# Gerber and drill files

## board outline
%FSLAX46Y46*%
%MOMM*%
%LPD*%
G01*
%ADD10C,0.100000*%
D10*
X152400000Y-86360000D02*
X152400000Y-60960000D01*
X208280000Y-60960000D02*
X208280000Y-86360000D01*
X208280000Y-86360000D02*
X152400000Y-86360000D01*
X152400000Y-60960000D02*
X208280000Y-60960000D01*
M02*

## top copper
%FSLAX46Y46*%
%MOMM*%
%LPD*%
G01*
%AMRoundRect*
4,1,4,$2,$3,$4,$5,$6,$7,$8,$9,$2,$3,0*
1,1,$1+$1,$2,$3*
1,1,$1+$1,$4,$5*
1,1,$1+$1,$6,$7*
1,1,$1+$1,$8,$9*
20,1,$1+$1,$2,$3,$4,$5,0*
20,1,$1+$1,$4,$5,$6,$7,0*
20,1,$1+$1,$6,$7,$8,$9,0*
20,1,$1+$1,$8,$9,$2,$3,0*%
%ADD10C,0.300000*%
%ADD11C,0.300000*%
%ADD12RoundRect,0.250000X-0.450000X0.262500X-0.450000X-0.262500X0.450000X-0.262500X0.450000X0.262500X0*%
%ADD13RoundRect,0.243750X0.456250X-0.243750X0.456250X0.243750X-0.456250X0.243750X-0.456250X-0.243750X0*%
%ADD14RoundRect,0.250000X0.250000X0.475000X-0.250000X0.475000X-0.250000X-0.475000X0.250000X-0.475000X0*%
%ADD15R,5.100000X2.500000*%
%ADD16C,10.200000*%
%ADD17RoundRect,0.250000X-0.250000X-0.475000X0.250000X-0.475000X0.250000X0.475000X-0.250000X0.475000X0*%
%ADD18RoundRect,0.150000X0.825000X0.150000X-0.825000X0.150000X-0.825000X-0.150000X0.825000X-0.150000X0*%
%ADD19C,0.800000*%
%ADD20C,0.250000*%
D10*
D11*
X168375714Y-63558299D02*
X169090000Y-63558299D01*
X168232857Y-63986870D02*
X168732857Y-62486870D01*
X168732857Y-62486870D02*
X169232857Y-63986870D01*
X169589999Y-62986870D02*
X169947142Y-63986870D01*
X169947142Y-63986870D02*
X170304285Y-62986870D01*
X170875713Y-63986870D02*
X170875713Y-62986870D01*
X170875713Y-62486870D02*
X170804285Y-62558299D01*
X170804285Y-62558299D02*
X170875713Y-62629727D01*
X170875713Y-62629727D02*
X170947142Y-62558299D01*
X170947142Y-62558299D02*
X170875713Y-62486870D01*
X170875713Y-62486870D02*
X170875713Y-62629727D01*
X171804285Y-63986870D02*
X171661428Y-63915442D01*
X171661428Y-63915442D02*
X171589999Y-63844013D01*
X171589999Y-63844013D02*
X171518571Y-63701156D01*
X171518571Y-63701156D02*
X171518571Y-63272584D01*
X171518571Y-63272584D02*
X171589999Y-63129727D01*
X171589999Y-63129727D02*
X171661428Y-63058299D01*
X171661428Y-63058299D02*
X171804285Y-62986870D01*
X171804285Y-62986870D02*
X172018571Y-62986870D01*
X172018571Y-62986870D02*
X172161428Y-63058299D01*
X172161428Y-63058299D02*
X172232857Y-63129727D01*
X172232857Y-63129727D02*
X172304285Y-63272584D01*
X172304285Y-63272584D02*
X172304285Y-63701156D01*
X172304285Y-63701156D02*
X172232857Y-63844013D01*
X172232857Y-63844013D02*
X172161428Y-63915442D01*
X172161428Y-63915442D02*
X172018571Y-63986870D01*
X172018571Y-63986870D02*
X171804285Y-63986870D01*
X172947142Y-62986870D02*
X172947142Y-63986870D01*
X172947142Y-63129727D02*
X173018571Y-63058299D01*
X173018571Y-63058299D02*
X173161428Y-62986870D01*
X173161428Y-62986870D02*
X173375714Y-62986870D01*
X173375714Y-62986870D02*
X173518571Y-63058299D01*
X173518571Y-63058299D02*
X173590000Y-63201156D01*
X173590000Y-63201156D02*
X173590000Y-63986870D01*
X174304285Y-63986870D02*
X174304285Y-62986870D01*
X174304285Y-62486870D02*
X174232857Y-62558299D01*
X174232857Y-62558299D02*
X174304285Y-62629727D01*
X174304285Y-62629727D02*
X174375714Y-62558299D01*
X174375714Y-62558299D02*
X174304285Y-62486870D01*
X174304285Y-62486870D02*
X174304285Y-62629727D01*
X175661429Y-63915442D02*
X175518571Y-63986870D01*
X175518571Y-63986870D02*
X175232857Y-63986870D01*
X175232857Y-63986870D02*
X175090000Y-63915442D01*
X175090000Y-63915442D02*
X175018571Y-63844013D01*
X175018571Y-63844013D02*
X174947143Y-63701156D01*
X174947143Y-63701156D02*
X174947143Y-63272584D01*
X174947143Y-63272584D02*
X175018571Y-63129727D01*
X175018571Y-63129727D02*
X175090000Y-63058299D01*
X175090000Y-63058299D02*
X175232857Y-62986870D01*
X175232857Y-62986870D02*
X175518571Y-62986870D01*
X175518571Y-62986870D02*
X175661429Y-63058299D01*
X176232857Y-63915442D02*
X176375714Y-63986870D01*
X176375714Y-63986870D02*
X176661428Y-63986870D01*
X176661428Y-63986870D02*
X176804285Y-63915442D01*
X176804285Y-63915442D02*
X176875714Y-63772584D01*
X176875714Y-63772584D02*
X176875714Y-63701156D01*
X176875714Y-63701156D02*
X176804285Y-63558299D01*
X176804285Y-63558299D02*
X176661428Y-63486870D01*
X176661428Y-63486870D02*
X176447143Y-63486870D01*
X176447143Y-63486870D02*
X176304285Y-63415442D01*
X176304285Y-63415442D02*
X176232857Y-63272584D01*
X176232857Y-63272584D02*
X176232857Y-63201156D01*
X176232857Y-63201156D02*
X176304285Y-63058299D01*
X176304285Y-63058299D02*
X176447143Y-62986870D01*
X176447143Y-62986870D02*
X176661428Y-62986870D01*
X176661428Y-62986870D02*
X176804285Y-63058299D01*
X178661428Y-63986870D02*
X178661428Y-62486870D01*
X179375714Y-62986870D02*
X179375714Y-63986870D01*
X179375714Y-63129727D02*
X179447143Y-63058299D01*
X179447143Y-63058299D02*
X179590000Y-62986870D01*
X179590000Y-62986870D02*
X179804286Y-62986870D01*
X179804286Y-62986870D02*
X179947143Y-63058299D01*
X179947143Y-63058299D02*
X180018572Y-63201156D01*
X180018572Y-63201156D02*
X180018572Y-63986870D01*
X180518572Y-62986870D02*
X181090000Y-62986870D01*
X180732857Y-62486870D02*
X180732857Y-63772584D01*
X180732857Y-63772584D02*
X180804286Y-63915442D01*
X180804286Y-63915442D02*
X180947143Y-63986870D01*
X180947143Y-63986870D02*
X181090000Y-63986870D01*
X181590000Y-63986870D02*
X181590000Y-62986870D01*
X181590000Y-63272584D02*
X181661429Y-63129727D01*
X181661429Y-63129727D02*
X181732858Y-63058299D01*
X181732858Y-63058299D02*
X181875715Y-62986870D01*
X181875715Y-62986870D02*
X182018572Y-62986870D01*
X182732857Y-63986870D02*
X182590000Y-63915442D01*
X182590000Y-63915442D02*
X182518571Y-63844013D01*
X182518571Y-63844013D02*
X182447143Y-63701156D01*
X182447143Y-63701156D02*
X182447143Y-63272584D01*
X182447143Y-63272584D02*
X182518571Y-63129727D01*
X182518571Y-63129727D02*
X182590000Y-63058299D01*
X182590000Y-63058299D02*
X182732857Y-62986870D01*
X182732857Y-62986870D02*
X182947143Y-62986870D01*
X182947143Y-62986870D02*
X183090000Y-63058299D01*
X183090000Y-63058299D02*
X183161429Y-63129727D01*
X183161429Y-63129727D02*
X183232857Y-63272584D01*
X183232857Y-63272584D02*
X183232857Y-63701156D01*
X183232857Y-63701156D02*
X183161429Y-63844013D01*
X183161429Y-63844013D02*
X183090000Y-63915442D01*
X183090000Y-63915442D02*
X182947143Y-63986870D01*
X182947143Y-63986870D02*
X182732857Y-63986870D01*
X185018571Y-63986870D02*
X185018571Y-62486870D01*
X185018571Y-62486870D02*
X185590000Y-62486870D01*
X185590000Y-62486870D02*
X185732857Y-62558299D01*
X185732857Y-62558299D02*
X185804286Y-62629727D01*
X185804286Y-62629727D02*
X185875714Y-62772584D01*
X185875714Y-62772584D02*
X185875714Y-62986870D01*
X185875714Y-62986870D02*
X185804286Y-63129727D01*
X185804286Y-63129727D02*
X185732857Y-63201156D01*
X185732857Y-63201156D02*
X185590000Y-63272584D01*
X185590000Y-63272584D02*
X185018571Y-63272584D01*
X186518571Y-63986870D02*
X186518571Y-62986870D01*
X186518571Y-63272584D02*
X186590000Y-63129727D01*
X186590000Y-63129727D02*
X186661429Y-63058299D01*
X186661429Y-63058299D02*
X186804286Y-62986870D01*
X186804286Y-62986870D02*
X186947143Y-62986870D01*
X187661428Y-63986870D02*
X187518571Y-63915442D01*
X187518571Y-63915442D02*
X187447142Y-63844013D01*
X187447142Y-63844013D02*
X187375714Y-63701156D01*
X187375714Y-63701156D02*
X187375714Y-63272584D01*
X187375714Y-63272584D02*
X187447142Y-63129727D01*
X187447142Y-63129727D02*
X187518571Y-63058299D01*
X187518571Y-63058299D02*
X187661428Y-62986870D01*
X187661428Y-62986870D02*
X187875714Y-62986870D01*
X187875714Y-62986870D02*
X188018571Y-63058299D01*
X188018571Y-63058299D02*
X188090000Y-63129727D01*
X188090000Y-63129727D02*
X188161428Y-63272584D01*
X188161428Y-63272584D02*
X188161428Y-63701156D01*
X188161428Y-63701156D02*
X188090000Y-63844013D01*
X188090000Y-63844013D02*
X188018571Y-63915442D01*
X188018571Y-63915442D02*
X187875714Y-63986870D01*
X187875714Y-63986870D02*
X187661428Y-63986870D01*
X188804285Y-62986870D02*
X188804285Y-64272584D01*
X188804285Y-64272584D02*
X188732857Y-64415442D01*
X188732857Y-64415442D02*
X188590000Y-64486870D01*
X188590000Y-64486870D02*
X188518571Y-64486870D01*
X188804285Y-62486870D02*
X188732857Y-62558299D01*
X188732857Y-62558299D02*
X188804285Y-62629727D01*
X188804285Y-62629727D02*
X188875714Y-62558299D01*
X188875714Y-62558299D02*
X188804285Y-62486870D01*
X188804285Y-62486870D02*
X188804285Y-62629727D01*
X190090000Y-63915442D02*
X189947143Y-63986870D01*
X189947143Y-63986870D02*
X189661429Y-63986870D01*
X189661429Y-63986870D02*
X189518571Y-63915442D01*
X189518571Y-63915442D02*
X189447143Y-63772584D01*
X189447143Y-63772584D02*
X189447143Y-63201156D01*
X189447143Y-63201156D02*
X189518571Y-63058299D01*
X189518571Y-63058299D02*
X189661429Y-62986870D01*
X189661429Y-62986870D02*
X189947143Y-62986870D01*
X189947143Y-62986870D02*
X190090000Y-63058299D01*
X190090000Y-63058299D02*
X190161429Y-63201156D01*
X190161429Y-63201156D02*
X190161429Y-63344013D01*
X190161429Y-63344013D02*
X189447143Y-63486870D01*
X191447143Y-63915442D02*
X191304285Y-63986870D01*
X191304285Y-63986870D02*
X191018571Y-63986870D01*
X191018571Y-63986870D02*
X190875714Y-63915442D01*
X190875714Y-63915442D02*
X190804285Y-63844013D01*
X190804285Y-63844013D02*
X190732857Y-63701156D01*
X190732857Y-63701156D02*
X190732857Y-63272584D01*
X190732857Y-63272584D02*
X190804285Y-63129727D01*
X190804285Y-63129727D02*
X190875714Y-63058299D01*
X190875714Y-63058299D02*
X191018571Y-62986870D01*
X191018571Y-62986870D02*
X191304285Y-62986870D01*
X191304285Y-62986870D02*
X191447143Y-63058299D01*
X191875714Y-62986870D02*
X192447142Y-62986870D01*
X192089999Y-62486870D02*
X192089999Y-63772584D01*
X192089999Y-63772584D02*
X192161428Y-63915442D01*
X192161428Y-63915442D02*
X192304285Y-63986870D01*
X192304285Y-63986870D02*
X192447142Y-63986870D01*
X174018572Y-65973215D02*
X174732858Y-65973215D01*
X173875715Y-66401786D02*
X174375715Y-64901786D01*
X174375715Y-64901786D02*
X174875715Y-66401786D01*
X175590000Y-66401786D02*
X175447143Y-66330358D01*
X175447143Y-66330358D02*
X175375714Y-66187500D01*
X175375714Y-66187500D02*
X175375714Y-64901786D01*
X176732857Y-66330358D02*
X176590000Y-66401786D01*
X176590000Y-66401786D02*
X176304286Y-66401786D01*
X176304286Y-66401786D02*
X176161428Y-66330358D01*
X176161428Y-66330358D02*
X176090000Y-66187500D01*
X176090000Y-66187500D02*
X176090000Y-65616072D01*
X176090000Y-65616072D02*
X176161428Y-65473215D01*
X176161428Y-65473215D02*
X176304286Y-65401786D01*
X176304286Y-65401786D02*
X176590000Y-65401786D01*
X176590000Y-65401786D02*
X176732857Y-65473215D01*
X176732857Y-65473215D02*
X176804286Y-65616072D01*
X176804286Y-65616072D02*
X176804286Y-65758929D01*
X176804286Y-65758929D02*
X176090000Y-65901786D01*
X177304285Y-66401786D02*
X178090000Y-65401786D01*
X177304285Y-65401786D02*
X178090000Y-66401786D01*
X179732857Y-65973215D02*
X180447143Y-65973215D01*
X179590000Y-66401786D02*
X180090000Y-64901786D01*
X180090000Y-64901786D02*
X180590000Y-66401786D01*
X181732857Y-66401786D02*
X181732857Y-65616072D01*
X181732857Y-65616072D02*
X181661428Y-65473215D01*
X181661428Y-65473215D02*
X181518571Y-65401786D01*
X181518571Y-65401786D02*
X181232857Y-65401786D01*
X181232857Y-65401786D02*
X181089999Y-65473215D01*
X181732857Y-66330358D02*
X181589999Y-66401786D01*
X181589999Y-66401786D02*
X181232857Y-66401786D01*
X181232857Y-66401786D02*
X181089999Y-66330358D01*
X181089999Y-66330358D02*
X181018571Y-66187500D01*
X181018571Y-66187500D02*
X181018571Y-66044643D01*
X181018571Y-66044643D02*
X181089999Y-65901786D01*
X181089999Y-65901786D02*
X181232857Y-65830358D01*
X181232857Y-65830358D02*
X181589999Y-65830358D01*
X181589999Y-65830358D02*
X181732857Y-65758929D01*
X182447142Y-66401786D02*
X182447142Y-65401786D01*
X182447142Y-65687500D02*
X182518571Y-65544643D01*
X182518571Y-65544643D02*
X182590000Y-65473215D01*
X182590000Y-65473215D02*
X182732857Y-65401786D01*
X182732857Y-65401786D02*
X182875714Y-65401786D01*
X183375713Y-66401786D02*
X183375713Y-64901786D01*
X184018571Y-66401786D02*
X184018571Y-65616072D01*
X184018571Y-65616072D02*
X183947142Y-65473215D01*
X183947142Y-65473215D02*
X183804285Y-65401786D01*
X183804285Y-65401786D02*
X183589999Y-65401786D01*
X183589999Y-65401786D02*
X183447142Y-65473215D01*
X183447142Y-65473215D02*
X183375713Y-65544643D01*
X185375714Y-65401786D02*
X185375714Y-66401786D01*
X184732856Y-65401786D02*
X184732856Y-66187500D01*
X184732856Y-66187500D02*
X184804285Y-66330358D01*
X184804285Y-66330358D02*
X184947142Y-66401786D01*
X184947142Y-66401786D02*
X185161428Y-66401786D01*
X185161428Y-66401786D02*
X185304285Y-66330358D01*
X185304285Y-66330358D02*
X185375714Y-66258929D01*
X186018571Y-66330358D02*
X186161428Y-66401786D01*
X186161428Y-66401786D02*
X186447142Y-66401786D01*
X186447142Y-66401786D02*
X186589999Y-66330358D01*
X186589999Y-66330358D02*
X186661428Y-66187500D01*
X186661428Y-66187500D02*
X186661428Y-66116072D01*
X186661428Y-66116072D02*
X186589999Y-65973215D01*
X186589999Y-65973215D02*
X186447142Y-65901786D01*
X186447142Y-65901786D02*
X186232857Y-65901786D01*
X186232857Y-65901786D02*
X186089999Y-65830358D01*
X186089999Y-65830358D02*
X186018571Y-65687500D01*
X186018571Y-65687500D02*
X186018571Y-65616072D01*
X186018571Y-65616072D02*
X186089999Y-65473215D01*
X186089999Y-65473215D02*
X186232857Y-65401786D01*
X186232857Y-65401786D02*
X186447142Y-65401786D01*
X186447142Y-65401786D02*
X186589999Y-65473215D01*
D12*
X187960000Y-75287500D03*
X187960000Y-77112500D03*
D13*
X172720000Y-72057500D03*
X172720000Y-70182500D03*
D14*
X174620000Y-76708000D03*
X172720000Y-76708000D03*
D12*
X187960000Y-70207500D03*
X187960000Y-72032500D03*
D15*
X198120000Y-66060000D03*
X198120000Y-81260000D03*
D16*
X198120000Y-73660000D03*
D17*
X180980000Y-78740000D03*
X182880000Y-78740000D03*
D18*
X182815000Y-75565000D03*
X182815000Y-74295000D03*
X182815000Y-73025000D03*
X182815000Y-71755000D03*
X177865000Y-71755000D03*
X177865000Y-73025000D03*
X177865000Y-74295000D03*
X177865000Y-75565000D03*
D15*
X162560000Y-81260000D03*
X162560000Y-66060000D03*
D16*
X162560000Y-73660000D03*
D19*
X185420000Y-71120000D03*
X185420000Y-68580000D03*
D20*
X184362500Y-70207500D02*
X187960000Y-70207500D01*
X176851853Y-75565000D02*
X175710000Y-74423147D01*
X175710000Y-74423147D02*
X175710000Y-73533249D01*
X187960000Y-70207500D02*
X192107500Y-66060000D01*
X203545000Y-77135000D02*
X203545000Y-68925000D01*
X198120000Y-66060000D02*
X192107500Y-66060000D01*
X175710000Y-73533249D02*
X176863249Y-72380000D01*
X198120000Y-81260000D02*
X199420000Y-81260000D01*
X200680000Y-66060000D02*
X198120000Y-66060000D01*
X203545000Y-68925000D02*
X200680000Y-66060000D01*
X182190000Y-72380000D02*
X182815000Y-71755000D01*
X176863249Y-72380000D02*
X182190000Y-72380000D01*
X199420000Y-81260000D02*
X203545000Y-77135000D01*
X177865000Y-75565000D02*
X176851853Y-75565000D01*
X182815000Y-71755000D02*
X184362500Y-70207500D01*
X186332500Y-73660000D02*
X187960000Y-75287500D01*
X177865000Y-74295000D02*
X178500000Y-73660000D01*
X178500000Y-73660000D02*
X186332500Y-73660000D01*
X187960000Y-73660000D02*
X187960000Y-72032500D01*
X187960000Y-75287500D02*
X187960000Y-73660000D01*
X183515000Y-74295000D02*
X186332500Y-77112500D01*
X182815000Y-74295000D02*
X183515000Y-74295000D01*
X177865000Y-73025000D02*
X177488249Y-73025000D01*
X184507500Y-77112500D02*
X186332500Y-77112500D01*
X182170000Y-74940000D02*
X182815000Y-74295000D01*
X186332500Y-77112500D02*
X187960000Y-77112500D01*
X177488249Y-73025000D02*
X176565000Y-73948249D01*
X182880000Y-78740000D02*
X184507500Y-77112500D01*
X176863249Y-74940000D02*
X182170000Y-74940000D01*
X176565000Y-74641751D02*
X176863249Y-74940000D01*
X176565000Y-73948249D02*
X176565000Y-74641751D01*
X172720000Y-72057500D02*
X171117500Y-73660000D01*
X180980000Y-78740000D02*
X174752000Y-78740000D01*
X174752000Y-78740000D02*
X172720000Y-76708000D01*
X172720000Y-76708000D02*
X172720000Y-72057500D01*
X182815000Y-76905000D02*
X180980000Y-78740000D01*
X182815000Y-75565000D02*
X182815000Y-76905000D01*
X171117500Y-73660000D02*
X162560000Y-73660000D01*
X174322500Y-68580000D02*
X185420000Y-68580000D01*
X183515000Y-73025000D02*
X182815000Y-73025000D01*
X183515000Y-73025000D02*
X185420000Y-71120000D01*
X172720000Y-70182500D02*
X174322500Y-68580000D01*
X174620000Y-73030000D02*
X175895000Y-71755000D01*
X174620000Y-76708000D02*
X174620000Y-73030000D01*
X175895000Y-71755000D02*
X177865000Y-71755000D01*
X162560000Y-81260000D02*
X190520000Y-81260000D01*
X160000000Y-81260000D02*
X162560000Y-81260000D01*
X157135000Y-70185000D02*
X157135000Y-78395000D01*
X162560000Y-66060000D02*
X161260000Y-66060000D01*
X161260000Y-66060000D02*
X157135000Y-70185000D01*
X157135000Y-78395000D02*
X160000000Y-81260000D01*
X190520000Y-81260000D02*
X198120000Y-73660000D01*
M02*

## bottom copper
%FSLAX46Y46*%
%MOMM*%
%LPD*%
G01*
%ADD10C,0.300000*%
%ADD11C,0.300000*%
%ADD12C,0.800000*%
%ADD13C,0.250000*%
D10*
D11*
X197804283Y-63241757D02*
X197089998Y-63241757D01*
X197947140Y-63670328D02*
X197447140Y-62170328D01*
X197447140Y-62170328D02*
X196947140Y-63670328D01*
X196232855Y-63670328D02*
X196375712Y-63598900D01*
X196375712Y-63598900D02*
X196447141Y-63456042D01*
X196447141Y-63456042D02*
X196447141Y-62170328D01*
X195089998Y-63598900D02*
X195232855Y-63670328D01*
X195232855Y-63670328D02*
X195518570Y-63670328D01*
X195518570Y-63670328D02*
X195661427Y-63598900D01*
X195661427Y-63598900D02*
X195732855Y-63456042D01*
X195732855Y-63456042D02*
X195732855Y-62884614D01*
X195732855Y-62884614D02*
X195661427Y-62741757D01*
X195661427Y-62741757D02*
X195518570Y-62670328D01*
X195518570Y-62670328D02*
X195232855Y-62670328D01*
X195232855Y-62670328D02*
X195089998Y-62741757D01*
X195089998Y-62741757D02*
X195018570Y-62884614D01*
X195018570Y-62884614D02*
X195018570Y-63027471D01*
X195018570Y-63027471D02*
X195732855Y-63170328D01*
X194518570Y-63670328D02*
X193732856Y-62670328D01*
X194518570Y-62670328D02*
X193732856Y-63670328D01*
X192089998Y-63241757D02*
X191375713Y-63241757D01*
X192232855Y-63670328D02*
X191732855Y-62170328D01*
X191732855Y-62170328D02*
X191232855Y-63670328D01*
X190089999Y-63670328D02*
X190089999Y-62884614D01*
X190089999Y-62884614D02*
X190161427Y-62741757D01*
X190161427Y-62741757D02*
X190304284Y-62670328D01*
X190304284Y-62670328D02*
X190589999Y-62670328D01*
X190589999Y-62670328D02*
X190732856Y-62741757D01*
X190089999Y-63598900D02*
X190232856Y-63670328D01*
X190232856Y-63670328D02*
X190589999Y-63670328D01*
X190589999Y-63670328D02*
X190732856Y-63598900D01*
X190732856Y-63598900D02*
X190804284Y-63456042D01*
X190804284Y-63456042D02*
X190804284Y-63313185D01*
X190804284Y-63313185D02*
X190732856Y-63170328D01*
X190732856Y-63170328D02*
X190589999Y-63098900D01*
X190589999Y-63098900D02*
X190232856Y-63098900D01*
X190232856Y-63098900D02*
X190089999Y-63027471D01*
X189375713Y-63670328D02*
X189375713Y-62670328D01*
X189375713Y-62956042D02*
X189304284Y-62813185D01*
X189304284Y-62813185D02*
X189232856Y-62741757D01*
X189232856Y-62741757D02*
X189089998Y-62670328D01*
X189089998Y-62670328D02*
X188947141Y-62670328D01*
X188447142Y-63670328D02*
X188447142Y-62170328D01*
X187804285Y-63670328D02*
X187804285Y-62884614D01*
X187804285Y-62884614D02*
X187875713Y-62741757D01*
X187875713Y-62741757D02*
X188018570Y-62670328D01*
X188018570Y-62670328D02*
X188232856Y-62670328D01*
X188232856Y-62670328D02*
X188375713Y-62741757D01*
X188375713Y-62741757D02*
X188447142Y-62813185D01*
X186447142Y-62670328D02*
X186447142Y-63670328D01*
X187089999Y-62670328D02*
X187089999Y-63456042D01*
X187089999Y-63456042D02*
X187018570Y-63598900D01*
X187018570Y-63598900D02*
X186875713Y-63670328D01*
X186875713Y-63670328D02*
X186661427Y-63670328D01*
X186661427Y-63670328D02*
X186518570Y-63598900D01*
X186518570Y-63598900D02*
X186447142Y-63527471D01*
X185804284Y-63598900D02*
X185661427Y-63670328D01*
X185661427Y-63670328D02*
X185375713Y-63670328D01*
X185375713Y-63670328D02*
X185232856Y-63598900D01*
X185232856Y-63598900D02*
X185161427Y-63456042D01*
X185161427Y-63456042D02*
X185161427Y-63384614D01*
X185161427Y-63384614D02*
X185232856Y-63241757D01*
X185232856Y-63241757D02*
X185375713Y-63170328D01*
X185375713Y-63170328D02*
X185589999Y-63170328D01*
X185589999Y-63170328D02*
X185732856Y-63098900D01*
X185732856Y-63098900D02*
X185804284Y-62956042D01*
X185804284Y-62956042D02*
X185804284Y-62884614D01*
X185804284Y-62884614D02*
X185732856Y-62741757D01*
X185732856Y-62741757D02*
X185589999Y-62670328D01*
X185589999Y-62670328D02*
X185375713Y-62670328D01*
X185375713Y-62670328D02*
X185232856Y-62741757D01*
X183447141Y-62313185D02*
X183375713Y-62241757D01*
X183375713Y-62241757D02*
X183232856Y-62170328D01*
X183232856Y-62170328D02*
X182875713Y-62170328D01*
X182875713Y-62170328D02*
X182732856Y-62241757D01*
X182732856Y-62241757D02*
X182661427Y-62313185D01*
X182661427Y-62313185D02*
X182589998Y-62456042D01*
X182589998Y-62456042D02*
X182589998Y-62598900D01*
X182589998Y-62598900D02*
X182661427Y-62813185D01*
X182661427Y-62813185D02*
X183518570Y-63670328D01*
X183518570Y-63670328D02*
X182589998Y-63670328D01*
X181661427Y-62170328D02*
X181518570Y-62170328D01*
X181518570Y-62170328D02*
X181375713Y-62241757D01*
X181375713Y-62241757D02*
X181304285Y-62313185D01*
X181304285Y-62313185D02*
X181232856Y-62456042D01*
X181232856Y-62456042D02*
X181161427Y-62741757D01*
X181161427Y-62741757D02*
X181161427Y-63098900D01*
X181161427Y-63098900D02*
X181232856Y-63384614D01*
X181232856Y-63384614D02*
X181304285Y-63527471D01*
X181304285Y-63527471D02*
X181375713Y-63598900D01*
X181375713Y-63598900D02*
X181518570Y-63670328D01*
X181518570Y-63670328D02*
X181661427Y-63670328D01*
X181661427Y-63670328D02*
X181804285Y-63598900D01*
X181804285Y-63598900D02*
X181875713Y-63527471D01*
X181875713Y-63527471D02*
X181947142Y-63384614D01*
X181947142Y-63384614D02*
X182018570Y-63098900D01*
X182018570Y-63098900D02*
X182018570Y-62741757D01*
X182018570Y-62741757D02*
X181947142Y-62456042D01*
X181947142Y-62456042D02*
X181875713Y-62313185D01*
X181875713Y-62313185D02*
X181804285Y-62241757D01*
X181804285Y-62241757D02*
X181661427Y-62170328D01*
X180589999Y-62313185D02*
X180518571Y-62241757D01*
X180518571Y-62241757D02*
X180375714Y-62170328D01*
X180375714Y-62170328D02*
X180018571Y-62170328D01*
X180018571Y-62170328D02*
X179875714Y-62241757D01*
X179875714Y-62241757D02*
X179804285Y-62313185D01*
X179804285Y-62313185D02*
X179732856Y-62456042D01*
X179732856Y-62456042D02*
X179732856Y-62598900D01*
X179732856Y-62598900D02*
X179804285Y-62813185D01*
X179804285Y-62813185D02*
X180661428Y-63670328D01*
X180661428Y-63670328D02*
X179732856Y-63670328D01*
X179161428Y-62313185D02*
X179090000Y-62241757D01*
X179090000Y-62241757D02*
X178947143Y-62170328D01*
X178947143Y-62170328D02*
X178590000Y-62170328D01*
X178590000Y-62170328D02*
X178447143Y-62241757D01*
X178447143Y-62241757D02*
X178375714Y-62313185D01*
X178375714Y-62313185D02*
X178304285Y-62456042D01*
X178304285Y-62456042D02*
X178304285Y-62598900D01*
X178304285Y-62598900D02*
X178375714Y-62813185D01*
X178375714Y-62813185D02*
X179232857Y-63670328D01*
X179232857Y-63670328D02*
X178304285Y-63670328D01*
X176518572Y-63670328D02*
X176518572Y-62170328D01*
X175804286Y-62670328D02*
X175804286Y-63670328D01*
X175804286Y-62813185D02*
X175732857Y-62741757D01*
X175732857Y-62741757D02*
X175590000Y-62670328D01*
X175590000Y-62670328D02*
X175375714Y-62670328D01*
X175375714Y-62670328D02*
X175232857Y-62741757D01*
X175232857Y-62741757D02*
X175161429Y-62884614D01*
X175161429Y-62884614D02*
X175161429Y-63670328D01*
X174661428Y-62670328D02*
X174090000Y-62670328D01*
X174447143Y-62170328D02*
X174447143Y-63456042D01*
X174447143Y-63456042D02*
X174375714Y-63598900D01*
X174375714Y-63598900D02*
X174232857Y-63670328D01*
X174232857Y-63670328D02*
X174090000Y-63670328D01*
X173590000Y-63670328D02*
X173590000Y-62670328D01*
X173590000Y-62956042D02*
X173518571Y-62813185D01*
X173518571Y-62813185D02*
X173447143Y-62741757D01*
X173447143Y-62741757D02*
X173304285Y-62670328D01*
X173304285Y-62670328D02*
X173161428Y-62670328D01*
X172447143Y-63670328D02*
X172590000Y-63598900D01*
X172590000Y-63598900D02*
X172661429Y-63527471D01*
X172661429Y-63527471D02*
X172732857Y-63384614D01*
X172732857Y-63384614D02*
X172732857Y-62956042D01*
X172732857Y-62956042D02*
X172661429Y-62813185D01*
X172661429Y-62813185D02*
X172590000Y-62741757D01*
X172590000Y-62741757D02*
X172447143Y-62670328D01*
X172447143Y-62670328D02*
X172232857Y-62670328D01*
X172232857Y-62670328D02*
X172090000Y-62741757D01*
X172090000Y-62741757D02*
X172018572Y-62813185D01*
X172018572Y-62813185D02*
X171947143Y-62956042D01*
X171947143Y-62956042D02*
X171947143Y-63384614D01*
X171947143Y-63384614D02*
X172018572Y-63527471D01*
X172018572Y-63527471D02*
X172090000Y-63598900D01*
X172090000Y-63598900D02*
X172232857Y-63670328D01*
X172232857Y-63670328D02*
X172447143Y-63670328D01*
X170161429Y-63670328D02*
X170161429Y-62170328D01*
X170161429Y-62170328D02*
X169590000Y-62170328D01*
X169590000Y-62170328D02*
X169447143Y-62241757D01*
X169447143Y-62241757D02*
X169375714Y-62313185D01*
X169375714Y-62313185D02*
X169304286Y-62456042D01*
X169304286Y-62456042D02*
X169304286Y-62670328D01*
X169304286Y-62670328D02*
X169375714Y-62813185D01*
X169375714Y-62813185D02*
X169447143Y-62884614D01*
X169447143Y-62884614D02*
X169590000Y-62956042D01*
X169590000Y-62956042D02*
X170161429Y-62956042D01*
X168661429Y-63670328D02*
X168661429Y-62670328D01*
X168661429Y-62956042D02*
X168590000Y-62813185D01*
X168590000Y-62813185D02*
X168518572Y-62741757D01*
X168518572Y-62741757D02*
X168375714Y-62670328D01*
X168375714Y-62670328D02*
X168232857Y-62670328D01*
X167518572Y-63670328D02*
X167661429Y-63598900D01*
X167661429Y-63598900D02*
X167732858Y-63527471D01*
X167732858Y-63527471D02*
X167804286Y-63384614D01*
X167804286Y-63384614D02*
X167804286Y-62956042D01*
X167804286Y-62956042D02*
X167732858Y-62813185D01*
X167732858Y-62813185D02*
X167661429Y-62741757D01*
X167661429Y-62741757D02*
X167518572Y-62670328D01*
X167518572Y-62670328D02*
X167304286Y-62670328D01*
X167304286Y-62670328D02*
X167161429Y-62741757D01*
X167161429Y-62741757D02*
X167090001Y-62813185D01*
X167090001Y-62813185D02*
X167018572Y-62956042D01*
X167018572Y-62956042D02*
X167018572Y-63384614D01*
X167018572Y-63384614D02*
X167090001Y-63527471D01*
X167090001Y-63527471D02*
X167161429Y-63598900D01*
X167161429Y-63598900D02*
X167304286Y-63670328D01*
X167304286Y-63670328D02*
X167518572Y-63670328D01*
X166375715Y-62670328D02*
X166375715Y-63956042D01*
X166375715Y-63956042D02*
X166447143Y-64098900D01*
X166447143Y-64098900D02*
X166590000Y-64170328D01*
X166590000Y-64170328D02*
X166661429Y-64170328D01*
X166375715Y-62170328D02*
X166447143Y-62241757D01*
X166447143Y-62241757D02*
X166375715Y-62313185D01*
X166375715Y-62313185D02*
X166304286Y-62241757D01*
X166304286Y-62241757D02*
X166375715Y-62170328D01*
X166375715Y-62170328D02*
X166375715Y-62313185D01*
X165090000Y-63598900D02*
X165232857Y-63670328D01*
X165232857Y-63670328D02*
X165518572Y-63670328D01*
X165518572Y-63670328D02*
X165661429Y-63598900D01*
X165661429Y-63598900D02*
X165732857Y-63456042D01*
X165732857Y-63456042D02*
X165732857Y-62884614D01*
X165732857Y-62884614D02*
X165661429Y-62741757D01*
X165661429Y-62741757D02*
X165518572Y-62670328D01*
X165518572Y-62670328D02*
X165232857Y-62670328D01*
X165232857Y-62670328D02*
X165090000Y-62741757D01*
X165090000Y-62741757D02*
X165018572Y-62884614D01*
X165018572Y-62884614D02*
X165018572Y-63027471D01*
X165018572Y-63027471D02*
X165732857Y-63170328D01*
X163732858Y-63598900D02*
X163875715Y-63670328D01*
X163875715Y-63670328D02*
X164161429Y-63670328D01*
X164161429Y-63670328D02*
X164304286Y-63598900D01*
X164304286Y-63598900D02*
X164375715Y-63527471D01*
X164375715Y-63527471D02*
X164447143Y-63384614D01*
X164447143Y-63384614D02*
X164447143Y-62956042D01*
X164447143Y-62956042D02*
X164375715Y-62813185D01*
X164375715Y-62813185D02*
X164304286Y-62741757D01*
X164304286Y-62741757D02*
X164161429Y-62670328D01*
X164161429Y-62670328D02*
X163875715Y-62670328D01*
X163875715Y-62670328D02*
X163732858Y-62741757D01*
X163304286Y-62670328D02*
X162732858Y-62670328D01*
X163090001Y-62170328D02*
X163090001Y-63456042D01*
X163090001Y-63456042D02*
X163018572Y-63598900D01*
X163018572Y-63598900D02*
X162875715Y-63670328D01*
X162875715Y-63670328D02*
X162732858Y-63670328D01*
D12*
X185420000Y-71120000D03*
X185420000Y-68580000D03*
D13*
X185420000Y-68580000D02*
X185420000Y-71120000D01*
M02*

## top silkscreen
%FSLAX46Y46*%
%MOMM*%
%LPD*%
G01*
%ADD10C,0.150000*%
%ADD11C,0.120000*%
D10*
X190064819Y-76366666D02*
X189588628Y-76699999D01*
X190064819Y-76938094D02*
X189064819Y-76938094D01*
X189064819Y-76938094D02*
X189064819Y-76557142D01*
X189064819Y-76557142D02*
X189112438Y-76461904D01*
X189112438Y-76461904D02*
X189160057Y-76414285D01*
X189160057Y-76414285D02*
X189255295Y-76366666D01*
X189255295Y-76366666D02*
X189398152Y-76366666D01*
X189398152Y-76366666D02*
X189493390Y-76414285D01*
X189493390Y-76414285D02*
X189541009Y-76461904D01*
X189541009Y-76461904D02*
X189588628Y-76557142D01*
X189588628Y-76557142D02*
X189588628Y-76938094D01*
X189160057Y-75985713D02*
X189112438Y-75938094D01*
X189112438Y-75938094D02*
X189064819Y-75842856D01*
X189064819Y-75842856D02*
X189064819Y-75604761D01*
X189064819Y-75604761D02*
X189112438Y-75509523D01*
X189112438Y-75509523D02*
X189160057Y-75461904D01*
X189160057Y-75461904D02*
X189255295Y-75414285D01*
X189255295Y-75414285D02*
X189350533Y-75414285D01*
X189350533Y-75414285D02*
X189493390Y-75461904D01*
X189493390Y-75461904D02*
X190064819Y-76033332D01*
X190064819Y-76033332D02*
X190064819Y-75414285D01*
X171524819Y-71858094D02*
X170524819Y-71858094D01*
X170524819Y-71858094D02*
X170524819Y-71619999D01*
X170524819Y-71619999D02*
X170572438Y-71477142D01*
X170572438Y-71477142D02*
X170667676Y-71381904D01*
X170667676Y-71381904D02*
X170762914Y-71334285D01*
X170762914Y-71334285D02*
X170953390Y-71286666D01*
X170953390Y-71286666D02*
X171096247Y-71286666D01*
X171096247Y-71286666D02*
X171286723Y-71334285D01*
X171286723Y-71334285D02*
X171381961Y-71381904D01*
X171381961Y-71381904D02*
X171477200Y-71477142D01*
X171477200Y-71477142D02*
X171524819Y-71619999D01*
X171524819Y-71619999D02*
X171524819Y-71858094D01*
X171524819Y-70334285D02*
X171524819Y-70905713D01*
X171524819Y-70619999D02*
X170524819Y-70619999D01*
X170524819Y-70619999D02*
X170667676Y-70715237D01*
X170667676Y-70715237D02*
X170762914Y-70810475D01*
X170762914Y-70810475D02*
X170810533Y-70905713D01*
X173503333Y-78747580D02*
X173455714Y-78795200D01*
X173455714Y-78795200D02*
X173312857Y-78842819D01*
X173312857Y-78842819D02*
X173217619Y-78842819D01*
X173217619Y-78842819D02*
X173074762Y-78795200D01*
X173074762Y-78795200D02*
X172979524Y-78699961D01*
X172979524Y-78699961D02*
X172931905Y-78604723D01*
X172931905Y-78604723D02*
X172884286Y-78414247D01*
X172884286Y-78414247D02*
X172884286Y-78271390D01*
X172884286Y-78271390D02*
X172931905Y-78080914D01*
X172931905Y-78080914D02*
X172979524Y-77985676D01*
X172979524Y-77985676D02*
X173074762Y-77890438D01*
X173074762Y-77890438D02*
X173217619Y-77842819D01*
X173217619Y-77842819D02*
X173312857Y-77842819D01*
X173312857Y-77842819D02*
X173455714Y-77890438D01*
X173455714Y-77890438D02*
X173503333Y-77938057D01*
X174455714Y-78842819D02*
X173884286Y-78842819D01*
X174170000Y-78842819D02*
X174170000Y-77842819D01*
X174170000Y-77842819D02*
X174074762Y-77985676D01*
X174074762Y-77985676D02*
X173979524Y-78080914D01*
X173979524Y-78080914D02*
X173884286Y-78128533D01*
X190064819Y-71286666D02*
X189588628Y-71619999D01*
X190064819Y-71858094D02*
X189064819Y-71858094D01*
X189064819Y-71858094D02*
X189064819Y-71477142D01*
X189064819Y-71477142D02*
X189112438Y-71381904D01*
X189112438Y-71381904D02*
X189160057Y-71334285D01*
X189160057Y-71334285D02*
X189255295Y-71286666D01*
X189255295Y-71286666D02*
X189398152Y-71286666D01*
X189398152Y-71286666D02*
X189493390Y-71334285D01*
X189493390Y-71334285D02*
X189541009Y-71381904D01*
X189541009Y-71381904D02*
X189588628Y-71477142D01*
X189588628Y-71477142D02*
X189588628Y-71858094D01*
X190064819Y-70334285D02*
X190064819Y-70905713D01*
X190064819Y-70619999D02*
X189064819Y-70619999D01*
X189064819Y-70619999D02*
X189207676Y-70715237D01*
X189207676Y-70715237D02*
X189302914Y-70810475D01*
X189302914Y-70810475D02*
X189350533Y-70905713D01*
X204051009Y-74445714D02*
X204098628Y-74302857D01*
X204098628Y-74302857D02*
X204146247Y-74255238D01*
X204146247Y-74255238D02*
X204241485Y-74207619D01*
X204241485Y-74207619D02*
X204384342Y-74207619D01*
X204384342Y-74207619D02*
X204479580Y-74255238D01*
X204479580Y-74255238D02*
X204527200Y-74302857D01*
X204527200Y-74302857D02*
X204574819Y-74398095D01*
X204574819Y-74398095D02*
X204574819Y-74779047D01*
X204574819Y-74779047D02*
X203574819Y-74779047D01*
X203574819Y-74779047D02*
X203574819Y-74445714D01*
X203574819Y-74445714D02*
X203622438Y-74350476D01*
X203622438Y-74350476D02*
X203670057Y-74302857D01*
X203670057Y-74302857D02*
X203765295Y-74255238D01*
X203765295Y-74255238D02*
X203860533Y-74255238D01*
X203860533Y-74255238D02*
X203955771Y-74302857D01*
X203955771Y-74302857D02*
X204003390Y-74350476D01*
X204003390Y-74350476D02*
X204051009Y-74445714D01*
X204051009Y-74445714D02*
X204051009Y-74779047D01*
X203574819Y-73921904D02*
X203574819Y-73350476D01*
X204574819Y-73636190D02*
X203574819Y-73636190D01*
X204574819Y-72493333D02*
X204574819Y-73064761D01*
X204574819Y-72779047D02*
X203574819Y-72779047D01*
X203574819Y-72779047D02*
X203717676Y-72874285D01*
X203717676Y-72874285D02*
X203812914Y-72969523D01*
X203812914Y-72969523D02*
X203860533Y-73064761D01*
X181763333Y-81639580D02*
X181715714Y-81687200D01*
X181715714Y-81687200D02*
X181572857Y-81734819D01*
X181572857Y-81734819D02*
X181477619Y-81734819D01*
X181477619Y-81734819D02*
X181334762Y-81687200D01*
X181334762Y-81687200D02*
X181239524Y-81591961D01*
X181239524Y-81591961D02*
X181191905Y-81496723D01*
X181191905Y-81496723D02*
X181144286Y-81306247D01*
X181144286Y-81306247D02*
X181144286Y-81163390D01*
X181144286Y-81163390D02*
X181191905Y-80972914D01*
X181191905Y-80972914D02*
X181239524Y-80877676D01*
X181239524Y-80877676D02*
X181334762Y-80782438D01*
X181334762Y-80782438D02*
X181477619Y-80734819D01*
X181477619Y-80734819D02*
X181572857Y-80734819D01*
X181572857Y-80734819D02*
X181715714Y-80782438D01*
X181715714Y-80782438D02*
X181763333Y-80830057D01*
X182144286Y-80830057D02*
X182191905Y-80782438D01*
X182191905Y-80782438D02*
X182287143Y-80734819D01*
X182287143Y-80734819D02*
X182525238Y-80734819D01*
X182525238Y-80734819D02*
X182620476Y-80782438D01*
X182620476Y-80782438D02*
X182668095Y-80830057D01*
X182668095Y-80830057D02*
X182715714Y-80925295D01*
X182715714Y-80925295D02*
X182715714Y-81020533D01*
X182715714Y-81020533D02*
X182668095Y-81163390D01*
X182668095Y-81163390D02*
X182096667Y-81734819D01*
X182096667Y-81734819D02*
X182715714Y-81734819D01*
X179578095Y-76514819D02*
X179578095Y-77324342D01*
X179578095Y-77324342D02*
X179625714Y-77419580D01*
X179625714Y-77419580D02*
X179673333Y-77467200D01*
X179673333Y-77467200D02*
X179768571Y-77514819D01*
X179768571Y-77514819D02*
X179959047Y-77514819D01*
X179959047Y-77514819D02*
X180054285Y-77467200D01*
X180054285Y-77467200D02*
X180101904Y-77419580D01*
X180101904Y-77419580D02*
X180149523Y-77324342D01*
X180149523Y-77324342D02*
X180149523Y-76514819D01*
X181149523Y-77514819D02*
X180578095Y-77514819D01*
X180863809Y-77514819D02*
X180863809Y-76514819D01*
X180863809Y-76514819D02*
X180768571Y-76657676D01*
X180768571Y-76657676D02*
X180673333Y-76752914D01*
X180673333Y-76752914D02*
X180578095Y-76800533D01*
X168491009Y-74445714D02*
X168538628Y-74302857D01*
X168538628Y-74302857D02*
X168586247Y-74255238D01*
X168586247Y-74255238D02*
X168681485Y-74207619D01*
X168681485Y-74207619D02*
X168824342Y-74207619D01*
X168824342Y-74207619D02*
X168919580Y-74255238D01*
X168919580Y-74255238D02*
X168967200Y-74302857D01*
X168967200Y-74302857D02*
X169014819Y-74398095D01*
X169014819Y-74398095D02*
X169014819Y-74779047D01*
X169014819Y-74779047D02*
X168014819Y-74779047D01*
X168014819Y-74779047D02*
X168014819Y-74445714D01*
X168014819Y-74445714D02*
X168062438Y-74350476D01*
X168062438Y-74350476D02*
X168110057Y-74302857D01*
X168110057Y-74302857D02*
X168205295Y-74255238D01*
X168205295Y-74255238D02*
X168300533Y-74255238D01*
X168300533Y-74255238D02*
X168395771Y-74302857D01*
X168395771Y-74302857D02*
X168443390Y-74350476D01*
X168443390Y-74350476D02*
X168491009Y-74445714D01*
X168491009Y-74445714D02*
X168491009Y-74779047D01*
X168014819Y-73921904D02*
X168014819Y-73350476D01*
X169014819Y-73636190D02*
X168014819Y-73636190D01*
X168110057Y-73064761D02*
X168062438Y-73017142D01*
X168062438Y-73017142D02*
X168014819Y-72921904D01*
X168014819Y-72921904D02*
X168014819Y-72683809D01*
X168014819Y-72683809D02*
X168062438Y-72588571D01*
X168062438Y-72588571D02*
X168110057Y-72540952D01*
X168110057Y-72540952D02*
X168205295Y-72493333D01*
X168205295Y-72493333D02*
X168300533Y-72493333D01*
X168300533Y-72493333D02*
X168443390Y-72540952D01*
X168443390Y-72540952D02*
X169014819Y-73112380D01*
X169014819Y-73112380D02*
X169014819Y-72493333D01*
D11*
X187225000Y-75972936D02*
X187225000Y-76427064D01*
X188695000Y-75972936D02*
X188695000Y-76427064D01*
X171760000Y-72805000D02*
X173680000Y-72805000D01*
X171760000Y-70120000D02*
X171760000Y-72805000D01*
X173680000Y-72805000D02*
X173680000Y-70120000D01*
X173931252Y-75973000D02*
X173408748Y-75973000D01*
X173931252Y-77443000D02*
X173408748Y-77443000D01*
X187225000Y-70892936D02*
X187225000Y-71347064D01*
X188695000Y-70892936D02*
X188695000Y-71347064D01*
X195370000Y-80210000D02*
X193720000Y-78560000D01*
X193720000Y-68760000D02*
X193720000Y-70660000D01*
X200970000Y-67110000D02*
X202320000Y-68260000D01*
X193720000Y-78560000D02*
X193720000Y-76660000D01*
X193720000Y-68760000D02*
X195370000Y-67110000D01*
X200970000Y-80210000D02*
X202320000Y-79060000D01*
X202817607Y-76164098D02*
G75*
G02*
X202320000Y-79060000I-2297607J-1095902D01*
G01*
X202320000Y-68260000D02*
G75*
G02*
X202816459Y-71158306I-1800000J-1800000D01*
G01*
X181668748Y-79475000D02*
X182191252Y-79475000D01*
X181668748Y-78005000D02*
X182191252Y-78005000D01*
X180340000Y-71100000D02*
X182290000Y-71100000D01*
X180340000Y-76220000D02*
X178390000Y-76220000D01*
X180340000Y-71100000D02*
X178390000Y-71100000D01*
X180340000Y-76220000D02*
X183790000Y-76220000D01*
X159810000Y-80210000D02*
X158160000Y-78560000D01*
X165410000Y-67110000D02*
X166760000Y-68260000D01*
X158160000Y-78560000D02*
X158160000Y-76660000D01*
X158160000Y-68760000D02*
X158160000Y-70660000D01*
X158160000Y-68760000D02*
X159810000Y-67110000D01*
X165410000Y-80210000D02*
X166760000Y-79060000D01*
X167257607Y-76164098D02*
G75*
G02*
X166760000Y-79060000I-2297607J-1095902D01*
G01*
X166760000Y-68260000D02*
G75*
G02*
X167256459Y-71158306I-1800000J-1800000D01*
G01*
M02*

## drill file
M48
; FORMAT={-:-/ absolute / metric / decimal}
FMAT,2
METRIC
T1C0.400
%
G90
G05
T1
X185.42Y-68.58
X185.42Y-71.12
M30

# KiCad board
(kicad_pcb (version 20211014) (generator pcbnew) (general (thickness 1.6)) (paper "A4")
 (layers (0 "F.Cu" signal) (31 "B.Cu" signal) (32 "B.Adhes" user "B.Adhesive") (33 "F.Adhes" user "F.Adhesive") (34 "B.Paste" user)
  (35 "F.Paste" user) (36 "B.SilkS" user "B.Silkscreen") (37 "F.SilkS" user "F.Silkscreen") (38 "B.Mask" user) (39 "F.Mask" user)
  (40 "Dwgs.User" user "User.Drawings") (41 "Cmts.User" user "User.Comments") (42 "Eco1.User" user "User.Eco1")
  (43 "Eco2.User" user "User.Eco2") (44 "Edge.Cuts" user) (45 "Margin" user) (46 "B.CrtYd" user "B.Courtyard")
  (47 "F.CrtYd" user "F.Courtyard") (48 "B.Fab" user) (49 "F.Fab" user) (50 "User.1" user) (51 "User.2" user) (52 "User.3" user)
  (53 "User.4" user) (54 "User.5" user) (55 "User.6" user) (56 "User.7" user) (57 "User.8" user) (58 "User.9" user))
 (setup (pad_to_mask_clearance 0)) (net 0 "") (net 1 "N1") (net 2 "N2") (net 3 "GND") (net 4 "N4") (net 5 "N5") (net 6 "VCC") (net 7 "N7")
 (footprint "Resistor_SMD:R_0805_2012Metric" (layer "F.Cu") (at 187.96 76.2 -90)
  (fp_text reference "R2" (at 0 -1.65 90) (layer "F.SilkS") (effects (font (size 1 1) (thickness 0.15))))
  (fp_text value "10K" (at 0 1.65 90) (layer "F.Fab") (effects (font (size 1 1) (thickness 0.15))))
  (fp_line (start -0.227064 0.735) (end 0.227064 0.735) (layer "F.SilkS") (width 0.12))
  (fp_line (start -0.227064 -0.735) (end 0.227064 -0.735) (layer "F.SilkS") (width 0.12))
  (pad "1" smd roundrect (at -0.9125 0 270) (size 1.025 1.4) (layers "F.Cu" "F.Paste" "F.Mask") (roundrect_rratio 0.243902439) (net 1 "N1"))
  (pad "2" smd roundrect (at 0.9125 0 270) (size 1.025 1.4) (layers "F.Cu" "F.Paste" "F.Mask") (roundrect_rratio 0.243902439) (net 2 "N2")))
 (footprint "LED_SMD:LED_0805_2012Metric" (layer "F.Cu") (at 172.72 71.12 90)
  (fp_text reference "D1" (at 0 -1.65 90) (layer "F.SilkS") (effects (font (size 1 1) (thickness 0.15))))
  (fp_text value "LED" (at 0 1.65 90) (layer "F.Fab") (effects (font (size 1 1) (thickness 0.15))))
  (fp_line (start -1.685 -0.96) (end -1.685 0.96) (layer "F.SilkS") (width 0.12))
  (fp_line (start 1 -0.96) (end -1.685 -0.96) (layer "F.SilkS") (width 0.12))
  (fp_line (start -1.685 0.96) (end 1 0.96) (layer "F.SilkS") (width 0.12))
  (pad "1" smd roundrect (at -0.9375 0 90) (size 0.975 1.4) (layers "F.Cu" "F.Paste" "F.Mask") (roundrect_rratio 0.25) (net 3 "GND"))
  (pad "2" smd roundrect (at 0.9375 0 90) (size 0.975 1.4) (layers "F.Cu" "F.Paste" "F.Mask") (roundrect_rratio 0.25) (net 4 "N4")))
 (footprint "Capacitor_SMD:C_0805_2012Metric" (layer "F.Cu") (at 173.67 76.708 180)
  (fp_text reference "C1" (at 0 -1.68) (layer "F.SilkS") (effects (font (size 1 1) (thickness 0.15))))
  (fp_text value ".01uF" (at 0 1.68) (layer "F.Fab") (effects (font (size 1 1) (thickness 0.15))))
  (fp_line (start -0.261252 0.735) (end 0.261252 0.735) (layer "F.SilkS") (width 0.12))
  (fp_line (start -0.261252 -0.735) (end 0.261252 -0.735) (layer "F.SilkS") (width 0.12))
  (pad "1" smd roundrect (at -0.95 0 180) (size 1 1.45) (layers "F.Cu" "F.Paste" "F.Mask") (roundrect_rratio 0.25) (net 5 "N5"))
  (pad "2" smd roundrect (at 0.95 0 180) (size 1 1.45) (layers "F.Cu" "F.Paste" "F.Mask") (roundrect_rratio 0.25) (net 3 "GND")))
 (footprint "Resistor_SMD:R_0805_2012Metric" (layer "F.Cu") (at 187.96 71.12 -90)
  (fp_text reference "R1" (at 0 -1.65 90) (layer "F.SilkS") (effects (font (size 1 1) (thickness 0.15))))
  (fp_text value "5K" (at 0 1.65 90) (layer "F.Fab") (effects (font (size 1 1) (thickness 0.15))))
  (fp_line (start -0.227064 0.735) (end 0.227064 0.735) (layer "F.SilkS") (width 0.12))
  (fp_line (start -0.227064 -0.735) (end 0.227064 -0.735) (layer "F.SilkS") (width 0.12))
  (pad "1" smd roundrect (at -0.9125 0 270) (size 1.025 1.4) (layers "F.Cu" "F.Paste" "F.Mask") (roundrect_rratio 0.243902439) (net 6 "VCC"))
  (pad "2" smd roundrect (at 0.9125 0 270) (size 1.025 1.4) (layers "F.Cu" "F.Paste" "F.Mask") (roundrect_rratio 0.243902439) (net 1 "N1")))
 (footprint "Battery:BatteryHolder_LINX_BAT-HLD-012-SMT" (layer "F.Cu") (at 198.12 73.66 90)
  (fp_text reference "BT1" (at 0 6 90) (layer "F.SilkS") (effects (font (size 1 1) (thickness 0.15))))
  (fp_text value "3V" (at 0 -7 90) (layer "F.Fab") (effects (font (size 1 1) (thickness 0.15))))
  (fp_line (start -6.55 -2.75) (end -4.9 -4.4) (layer "F.SilkS") (width 0.12))
  (fp_line (start 4.9 -4.4) (end 3 -4.4) (layer "F.SilkS") (width 0.12))
  (fp_line (start 6.55 2.85) (end 5.4 4.2) (layer "F.SilkS") (width 0.12))
  (fp_line (start -4.9 -4.4) (end -3 -4.4) (layer "F.SilkS") (width 0.12))
  (fp_line (start 4.9 -4.4) (end 6.55 -2.75) (layer "F.SilkS") (width 0.12))
  (fp_line (start -6.55 2.85) (end -5.4 4.2) (layer "F.SilkS") (width 0.12))
  (fp_arc (start -2.504098 4.697607) (mid -4.031094 4.908816) (end -5.4 4.2) (layer "F.SilkS") (width 0.12))
  (fp_arc (start 5.4 4.2) (mid 4.029781 4.909041) (end 2.501694 4.696459) (layer "F.SilkS") (width 0.12))
  (pad "1" smd rect (at 7.6 0 90) (size 2.5 5.1) (layers "F.Cu" "F.Paste" "F.Mask") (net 6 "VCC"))
  (pad "1" smd rect (at -7.6 0 90) (size 2.5 5.1) (layers "F.Cu" "F.Paste" "F.Mask") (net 6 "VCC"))
  (pad "2" smd circle (at 0 0 90) (size 10.2 10.2) (layers "F.Cu" "F.Mask") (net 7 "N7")))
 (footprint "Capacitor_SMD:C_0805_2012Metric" (layer "F.Cu") (at 181.93 78.74)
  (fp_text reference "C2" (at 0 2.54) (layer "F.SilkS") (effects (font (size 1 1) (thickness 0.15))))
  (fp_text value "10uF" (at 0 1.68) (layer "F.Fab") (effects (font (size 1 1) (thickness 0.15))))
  (fp_line (start -0.261252 0.735) (end 0.261252 0.735) (layer "F.SilkS") (width 0.12))
  (fp_line (start -0.261252 -0.735) (end 0.261252 -0.735) (layer "F.SilkS") (width 0.12))
  (pad "1" smd roundrect (at -0.95 0) (size 1 1.45) (layers "F.Cu" "F.Paste" "F.Mask") (roundrect_rratio 0.25) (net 3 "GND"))
  (pad "2" smd roundrect (at 0.95 0) (size 1 1.45) (layers "F.Cu" "F.Paste" "F.Mask") (roundrect_rratio 0.25) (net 2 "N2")))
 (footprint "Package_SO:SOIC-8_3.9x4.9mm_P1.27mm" (layer "F.Cu") (at 180.34 73.66 180)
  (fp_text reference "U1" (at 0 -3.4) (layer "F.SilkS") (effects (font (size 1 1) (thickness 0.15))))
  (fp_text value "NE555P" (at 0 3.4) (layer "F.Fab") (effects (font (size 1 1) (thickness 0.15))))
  (fp_line (start 0 2.56) (end -1.95 2.56) (layer "F.SilkS") (width 0.12))
  (fp_line (start 0 -2.56) (end 1.95 -2.56) (layer "F.SilkS") (width 0.12))
  (fp_line (start 0 2.56) (end 1.95 2.56) (layer "F.SilkS") (width 0.12))
  (fp_line (start 0 -2.56) (end -3.45 -2.56) (layer "F.SilkS") (width 0.12))
  (pad "1" smd roundrect (at -2.475 -1.905 180) (size 1.95 0.6) (layers "F.Cu" "F.Paste" "F.Mask") (roundrect_rratio 0.25) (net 3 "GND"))
  (pad "2" smd roundrect (at -2.475 -0.635 180) (size 1.95 0.6) (layers "F.Cu" "F.Paste" "F.Mask") (roundrect_rratio 0.25) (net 2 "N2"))
  (pad "3" smd roundrect (at -2.475 0.635 180) (size 1.95 0.6) (layers "F.Cu" "F.Paste" "F.Mask") (roundrect_rratio 0.25) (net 4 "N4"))
  (pad "4" smd roundrect (at -2.475 1.905 180) (size 1.95 0.6) (layers "F.Cu" "F.Paste" "F.Mask") (roundrect_rratio 0.25) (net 6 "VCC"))
  (pad "5" smd roundrect (at 2.475 1.905 180) (size 1.95 0.6) (layers "F.Cu" "F.Paste" "F.Mask") (roundrect_rratio 0.25) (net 5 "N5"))
  (pad "6" smd roundrect (at 2.475 0.635 180) (size 1.95 0.6) (layers "F.Cu" "F.Paste" "F.Mask") (roundrect_rratio 0.25) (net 2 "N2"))
  (pad "7" smd roundrect (at 2.475 -0.635 180) (size 1.95 0.6) (layers "F.Cu" "F.Paste" "F.Mask") (roundrect_rratio 0.25) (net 1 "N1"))
  (pad "8" smd roundrect (at 2.475 -1.905 180) (size 1.95 0.6) (layers "F.Cu" "F.Paste" "F.Mask") (roundrect_rratio 0.25) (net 6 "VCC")))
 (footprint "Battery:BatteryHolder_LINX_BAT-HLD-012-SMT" (layer "F.Cu") (at 162.56 73.66 90)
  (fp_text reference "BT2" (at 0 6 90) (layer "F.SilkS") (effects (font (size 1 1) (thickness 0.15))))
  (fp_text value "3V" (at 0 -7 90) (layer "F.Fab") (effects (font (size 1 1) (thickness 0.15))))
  (fp_line (start -6.55 -2.75) (end -4.9 -4.4) (layer "F.SilkS") (width 0.12))
  (fp_line (start 6.55 2.85) (end 5.4 4.2) (layer "F.SilkS") (width 0.12))
  (fp_line (start -4.9 -4.4) (end -3 -4.4) (layer "F.SilkS") (width 0.12))
  (fp_line (start 4.9 -4.4) (end 3 -4.4) (layer "F.SilkS") (width 0.12))
  (fp_line (start 4.9 -4.4) (end 6.55 -2.75) (layer "F.SilkS") (width 0.12))
  (fp_line (start -6.55 2.85) (end -5.4 4.2) (layer "F.SilkS") (width 0.12))
  (fp_arc (start -2.504098 4.697607) (mid -4.031094 4.908816) (end -5.4 4.2) (layer "F.SilkS") (width 0.12))
  (fp_arc (start 5.4 4.2) (mid 4.029781 4.909041) (end 2.501694 4.696459) (layer "F.SilkS") (width 0.12))
  (pad "1" smd rect (at -7.6 0 90) (size 2.5 5.1) (layers "F.Cu" "F.Paste" "F.Mask") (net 7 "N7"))
  (pad "1" smd rect (at 7.6 0 90) (size 2.5 5.1) (layers "F.Cu" "F.Paste" "F.Mask") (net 7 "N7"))
  (pad "2" smd circle (at 0 0 90) (size 10.2 10.2) (layers "F.Cu" "F.Mask") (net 3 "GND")))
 (gr_line (start 152.4 86.36) (end 152.4 60.96) (layer "Edge.Cuts") (width 0.1))
 (gr_line (start 208.28 60.96) (end 208.28 86.36) (layer "Edge.Cuts") (width 0.1))
 (gr_line (start 208.28 86.36) (end 152.4 86.36) (layer "Edge.Cuts") (width 0.1))
 (gr_line (start 152.4 60.96) (end 208.28 60.96) (layer "Edge.Cuts") (width 0.1))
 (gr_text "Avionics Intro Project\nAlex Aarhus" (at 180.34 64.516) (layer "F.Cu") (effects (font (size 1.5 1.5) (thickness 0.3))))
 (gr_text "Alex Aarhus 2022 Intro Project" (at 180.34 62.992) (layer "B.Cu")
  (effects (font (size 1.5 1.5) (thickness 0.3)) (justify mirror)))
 (segment (start 184.3625 70.2075) (end 187.96 70.2075) (width 0.25) (layer "F.Cu") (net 6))
 (segment (start 176.851853 75.565) (end 175.71 74.423147) (width 0.25) (layer "F.Cu") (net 6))
 (segment (start 175.71 74.423147) (end 175.71 73.533249) (width 0.25) (layer "F.Cu") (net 6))
 (segment (start 187.96 70.2075) (end 192.1075 66.06) (width 0.25) (layer "F.Cu") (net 6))
 (segment (start 203.545 77.135) (end 203.545 68.925) (width 0.25) (layer "F.Cu") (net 6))
 (segment (start 198.12 66.06) (end 192.1075 66.06) (width 0.25) (layer "F.Cu") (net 6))
 (segment (start 175.71 73.533249) (end 176.863249 72.38) (width 0.25) (layer "F.Cu") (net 6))
 (segment (start 198.12 81.26) (end 199.42 81.26) (width 0.25) (layer "F.Cu") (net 6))
 (segment (start 200.68 66.06) (end 198.12 66.06) (width 0.25) (layer "F.Cu") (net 6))
 (segment (start 203.545 68.925) (end 200.68 66.06) (width 0.25) (layer "F.Cu") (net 6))
 (segment (start 182.19 72.38) (end 182.815 71.755) (width 0.25) (layer "F.Cu") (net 6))
 (segment (start 176.863249 72.38) (end 182.19 72.38) (width 0.25) (layer "F.Cu") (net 6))
 (segment (start 199.42 81.26) (end 203.545 77.135) (width 0.25) (layer "F.Cu") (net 6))
 (segment (start 177.865 75.565) (end 176.851853 75.565) (width 0.25) (layer "F.Cu") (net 6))
 (segment (start 182.815 71.755) (end 184.3625 70.2075) (width 0.25) (layer "F.Cu") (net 6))
 (segment (start 186.3325 73.66) (end 187.96 75.2875) (width 0.25) (layer "F.Cu") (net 1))
 (segment (start 177.865 74.295) (end 178.5 73.66) (width 0.25) (layer "F.Cu") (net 1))
 (segment (start 178.5 73.66) (end 186.3325 73.66) (width 0.25) (layer "F.Cu") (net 1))
 (segment (start 187.96 73.66) (end 187.96 72.0325) (width 0.25) (layer "F.Cu") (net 1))
 (segment (start 187.96 75.2875) (end 187.96 73.66) (width 0.25) (layer "F.Cu") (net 1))
 (segment (start 183.515 74.295) (end 186.3325 77.1125) (width 0.25) (layer "F.Cu") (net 2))
 (segment (start 182.815 74.295) (end 183.515 74.295) (width 0.25) (layer "F.Cu") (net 2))
 (segment (start 177.865 73.025) (end 177.488249 73.025) (width 0.25) (layer "F.Cu") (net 2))
 (segment (start 184.5075 77.1125) (end 186.3325 77.1125) (width 0.25) (layer "F.Cu") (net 2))
 (segment (start 182.17 74.94) (end 182.815 74.295) (width 0.25) (layer "F.Cu") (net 2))
 (segment (start 186.3325 77.1125) (end 187.96 77.1125) (width 0.25) (layer "F.Cu") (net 2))
 (segment (start 177.488249 73.025) (end 176.565 73.948249) (width 0.25) (layer "F.Cu") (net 2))
 (segment (start 182.88 78.74) (end 184.5075 77.1125) (width 0.25) (layer "F.Cu") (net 2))
 (segment (start 176.863249 74.94) (end 182.17 74.94) (width 0.25) (layer "F.Cu") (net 2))
 (segment (start 176.565 74.641751) (end 176.863249 74.94) (width 0.25) (layer "F.Cu") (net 2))
 (segment (start 176.565 73.948249) (end 176.565 74.641751) (width 0.25) (layer "F.Cu") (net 2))
 (segment (start 172.72 72.0575) (end 171.1175 73.66) (width 0.25) (layer "F.Cu") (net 3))
 (segment (start 180.98 78.74) (end 174.752 78.74) (width 0.25) (layer "F.Cu") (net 3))
 (segment (start 174.752 78.74) (end 172.72 76.708) (width 0.25) (layer "F.Cu") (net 3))
 (segment (start 172.72 76.708) (end 172.72 72.0575) (width 0.25) (layer "F.Cu") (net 3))
 (segment (start 182.815 76.905) (end 180.98 78.74) (width 0.25) (layer "F.Cu") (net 3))
 (segment (start 182.815 75.565) (end 182.815 76.905) (width 0.25) (layer "F.Cu") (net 3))
 (segment (start 171.1175 73.66) (end 162.56 73.66) (width 0.25) (layer "F.Cu") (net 3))
 (segment (start 174.3225 68.58) (end 185.42 68.58) (width 0.25) (layer "F.Cu") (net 4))
 (segment (start 183.515 73.025) (end 182.815 73.025) (width 0.25) (layer "F.Cu") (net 4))
 (segment (start 183.515 73.025) (end 185.42 71.12) (width 0.25) (layer "F.Cu") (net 4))
 (segment (start 172.72 70.1825) (end 174.3225 68.58) (width 0.25) (layer "F.Cu") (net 4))
 (via (at 185.42 71.12) (size 0.8) (drill 0.4) (layers "F.Cu" "B.Cu") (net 4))
 (via (at 185.42 68.58) (size 0.8) (drill 0.4) (layers "F.Cu" "B.Cu") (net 4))
 (segment (start 185.42 68.58) (end 185.42 71.12) (width 0.25) (layer "B.Cu") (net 4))
 (segment (start 174.62 73.03) (end 175.895 71.755) (width 0.25) (layer "F.Cu") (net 5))
 (segment (start 174.62 76.708) (end 174.62 73.03) (width 0.25) (layer "F.Cu") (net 5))
 (segment (start 175.895 71.755) (end 177.865 71.755) (width 0.25) (layer "F.Cu") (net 5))
 (segment (start 162.56 81.26) (end 190.52 81.26) (width 0.25) (layer "F.Cu") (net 7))
 (segment (start 160 81.26) (end 162.56 81.26) (width 0.25) (layer "F.Cu") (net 7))
 (segment (start 157.135 70.185) (end 157.135 78.395) (width 0.25) (layer "F.Cu") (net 7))
 (segment (start 162.56 66.06) (end 161.26 66.06) (width 0.25) (layer "F.Cu") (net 7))
 (segment (start 161.26 66.06) (end 157.135 70.185) (width 0.25) (layer "F.Cu") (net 7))
 (segment (start 157.135 78.395) (end 160 81.26) (width 0.25) (layer "F.Cu") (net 7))
 (segment (start 190.52 81.26) (end 198.12 73.66) (width 0.25) (layer "F.Cu") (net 7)))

